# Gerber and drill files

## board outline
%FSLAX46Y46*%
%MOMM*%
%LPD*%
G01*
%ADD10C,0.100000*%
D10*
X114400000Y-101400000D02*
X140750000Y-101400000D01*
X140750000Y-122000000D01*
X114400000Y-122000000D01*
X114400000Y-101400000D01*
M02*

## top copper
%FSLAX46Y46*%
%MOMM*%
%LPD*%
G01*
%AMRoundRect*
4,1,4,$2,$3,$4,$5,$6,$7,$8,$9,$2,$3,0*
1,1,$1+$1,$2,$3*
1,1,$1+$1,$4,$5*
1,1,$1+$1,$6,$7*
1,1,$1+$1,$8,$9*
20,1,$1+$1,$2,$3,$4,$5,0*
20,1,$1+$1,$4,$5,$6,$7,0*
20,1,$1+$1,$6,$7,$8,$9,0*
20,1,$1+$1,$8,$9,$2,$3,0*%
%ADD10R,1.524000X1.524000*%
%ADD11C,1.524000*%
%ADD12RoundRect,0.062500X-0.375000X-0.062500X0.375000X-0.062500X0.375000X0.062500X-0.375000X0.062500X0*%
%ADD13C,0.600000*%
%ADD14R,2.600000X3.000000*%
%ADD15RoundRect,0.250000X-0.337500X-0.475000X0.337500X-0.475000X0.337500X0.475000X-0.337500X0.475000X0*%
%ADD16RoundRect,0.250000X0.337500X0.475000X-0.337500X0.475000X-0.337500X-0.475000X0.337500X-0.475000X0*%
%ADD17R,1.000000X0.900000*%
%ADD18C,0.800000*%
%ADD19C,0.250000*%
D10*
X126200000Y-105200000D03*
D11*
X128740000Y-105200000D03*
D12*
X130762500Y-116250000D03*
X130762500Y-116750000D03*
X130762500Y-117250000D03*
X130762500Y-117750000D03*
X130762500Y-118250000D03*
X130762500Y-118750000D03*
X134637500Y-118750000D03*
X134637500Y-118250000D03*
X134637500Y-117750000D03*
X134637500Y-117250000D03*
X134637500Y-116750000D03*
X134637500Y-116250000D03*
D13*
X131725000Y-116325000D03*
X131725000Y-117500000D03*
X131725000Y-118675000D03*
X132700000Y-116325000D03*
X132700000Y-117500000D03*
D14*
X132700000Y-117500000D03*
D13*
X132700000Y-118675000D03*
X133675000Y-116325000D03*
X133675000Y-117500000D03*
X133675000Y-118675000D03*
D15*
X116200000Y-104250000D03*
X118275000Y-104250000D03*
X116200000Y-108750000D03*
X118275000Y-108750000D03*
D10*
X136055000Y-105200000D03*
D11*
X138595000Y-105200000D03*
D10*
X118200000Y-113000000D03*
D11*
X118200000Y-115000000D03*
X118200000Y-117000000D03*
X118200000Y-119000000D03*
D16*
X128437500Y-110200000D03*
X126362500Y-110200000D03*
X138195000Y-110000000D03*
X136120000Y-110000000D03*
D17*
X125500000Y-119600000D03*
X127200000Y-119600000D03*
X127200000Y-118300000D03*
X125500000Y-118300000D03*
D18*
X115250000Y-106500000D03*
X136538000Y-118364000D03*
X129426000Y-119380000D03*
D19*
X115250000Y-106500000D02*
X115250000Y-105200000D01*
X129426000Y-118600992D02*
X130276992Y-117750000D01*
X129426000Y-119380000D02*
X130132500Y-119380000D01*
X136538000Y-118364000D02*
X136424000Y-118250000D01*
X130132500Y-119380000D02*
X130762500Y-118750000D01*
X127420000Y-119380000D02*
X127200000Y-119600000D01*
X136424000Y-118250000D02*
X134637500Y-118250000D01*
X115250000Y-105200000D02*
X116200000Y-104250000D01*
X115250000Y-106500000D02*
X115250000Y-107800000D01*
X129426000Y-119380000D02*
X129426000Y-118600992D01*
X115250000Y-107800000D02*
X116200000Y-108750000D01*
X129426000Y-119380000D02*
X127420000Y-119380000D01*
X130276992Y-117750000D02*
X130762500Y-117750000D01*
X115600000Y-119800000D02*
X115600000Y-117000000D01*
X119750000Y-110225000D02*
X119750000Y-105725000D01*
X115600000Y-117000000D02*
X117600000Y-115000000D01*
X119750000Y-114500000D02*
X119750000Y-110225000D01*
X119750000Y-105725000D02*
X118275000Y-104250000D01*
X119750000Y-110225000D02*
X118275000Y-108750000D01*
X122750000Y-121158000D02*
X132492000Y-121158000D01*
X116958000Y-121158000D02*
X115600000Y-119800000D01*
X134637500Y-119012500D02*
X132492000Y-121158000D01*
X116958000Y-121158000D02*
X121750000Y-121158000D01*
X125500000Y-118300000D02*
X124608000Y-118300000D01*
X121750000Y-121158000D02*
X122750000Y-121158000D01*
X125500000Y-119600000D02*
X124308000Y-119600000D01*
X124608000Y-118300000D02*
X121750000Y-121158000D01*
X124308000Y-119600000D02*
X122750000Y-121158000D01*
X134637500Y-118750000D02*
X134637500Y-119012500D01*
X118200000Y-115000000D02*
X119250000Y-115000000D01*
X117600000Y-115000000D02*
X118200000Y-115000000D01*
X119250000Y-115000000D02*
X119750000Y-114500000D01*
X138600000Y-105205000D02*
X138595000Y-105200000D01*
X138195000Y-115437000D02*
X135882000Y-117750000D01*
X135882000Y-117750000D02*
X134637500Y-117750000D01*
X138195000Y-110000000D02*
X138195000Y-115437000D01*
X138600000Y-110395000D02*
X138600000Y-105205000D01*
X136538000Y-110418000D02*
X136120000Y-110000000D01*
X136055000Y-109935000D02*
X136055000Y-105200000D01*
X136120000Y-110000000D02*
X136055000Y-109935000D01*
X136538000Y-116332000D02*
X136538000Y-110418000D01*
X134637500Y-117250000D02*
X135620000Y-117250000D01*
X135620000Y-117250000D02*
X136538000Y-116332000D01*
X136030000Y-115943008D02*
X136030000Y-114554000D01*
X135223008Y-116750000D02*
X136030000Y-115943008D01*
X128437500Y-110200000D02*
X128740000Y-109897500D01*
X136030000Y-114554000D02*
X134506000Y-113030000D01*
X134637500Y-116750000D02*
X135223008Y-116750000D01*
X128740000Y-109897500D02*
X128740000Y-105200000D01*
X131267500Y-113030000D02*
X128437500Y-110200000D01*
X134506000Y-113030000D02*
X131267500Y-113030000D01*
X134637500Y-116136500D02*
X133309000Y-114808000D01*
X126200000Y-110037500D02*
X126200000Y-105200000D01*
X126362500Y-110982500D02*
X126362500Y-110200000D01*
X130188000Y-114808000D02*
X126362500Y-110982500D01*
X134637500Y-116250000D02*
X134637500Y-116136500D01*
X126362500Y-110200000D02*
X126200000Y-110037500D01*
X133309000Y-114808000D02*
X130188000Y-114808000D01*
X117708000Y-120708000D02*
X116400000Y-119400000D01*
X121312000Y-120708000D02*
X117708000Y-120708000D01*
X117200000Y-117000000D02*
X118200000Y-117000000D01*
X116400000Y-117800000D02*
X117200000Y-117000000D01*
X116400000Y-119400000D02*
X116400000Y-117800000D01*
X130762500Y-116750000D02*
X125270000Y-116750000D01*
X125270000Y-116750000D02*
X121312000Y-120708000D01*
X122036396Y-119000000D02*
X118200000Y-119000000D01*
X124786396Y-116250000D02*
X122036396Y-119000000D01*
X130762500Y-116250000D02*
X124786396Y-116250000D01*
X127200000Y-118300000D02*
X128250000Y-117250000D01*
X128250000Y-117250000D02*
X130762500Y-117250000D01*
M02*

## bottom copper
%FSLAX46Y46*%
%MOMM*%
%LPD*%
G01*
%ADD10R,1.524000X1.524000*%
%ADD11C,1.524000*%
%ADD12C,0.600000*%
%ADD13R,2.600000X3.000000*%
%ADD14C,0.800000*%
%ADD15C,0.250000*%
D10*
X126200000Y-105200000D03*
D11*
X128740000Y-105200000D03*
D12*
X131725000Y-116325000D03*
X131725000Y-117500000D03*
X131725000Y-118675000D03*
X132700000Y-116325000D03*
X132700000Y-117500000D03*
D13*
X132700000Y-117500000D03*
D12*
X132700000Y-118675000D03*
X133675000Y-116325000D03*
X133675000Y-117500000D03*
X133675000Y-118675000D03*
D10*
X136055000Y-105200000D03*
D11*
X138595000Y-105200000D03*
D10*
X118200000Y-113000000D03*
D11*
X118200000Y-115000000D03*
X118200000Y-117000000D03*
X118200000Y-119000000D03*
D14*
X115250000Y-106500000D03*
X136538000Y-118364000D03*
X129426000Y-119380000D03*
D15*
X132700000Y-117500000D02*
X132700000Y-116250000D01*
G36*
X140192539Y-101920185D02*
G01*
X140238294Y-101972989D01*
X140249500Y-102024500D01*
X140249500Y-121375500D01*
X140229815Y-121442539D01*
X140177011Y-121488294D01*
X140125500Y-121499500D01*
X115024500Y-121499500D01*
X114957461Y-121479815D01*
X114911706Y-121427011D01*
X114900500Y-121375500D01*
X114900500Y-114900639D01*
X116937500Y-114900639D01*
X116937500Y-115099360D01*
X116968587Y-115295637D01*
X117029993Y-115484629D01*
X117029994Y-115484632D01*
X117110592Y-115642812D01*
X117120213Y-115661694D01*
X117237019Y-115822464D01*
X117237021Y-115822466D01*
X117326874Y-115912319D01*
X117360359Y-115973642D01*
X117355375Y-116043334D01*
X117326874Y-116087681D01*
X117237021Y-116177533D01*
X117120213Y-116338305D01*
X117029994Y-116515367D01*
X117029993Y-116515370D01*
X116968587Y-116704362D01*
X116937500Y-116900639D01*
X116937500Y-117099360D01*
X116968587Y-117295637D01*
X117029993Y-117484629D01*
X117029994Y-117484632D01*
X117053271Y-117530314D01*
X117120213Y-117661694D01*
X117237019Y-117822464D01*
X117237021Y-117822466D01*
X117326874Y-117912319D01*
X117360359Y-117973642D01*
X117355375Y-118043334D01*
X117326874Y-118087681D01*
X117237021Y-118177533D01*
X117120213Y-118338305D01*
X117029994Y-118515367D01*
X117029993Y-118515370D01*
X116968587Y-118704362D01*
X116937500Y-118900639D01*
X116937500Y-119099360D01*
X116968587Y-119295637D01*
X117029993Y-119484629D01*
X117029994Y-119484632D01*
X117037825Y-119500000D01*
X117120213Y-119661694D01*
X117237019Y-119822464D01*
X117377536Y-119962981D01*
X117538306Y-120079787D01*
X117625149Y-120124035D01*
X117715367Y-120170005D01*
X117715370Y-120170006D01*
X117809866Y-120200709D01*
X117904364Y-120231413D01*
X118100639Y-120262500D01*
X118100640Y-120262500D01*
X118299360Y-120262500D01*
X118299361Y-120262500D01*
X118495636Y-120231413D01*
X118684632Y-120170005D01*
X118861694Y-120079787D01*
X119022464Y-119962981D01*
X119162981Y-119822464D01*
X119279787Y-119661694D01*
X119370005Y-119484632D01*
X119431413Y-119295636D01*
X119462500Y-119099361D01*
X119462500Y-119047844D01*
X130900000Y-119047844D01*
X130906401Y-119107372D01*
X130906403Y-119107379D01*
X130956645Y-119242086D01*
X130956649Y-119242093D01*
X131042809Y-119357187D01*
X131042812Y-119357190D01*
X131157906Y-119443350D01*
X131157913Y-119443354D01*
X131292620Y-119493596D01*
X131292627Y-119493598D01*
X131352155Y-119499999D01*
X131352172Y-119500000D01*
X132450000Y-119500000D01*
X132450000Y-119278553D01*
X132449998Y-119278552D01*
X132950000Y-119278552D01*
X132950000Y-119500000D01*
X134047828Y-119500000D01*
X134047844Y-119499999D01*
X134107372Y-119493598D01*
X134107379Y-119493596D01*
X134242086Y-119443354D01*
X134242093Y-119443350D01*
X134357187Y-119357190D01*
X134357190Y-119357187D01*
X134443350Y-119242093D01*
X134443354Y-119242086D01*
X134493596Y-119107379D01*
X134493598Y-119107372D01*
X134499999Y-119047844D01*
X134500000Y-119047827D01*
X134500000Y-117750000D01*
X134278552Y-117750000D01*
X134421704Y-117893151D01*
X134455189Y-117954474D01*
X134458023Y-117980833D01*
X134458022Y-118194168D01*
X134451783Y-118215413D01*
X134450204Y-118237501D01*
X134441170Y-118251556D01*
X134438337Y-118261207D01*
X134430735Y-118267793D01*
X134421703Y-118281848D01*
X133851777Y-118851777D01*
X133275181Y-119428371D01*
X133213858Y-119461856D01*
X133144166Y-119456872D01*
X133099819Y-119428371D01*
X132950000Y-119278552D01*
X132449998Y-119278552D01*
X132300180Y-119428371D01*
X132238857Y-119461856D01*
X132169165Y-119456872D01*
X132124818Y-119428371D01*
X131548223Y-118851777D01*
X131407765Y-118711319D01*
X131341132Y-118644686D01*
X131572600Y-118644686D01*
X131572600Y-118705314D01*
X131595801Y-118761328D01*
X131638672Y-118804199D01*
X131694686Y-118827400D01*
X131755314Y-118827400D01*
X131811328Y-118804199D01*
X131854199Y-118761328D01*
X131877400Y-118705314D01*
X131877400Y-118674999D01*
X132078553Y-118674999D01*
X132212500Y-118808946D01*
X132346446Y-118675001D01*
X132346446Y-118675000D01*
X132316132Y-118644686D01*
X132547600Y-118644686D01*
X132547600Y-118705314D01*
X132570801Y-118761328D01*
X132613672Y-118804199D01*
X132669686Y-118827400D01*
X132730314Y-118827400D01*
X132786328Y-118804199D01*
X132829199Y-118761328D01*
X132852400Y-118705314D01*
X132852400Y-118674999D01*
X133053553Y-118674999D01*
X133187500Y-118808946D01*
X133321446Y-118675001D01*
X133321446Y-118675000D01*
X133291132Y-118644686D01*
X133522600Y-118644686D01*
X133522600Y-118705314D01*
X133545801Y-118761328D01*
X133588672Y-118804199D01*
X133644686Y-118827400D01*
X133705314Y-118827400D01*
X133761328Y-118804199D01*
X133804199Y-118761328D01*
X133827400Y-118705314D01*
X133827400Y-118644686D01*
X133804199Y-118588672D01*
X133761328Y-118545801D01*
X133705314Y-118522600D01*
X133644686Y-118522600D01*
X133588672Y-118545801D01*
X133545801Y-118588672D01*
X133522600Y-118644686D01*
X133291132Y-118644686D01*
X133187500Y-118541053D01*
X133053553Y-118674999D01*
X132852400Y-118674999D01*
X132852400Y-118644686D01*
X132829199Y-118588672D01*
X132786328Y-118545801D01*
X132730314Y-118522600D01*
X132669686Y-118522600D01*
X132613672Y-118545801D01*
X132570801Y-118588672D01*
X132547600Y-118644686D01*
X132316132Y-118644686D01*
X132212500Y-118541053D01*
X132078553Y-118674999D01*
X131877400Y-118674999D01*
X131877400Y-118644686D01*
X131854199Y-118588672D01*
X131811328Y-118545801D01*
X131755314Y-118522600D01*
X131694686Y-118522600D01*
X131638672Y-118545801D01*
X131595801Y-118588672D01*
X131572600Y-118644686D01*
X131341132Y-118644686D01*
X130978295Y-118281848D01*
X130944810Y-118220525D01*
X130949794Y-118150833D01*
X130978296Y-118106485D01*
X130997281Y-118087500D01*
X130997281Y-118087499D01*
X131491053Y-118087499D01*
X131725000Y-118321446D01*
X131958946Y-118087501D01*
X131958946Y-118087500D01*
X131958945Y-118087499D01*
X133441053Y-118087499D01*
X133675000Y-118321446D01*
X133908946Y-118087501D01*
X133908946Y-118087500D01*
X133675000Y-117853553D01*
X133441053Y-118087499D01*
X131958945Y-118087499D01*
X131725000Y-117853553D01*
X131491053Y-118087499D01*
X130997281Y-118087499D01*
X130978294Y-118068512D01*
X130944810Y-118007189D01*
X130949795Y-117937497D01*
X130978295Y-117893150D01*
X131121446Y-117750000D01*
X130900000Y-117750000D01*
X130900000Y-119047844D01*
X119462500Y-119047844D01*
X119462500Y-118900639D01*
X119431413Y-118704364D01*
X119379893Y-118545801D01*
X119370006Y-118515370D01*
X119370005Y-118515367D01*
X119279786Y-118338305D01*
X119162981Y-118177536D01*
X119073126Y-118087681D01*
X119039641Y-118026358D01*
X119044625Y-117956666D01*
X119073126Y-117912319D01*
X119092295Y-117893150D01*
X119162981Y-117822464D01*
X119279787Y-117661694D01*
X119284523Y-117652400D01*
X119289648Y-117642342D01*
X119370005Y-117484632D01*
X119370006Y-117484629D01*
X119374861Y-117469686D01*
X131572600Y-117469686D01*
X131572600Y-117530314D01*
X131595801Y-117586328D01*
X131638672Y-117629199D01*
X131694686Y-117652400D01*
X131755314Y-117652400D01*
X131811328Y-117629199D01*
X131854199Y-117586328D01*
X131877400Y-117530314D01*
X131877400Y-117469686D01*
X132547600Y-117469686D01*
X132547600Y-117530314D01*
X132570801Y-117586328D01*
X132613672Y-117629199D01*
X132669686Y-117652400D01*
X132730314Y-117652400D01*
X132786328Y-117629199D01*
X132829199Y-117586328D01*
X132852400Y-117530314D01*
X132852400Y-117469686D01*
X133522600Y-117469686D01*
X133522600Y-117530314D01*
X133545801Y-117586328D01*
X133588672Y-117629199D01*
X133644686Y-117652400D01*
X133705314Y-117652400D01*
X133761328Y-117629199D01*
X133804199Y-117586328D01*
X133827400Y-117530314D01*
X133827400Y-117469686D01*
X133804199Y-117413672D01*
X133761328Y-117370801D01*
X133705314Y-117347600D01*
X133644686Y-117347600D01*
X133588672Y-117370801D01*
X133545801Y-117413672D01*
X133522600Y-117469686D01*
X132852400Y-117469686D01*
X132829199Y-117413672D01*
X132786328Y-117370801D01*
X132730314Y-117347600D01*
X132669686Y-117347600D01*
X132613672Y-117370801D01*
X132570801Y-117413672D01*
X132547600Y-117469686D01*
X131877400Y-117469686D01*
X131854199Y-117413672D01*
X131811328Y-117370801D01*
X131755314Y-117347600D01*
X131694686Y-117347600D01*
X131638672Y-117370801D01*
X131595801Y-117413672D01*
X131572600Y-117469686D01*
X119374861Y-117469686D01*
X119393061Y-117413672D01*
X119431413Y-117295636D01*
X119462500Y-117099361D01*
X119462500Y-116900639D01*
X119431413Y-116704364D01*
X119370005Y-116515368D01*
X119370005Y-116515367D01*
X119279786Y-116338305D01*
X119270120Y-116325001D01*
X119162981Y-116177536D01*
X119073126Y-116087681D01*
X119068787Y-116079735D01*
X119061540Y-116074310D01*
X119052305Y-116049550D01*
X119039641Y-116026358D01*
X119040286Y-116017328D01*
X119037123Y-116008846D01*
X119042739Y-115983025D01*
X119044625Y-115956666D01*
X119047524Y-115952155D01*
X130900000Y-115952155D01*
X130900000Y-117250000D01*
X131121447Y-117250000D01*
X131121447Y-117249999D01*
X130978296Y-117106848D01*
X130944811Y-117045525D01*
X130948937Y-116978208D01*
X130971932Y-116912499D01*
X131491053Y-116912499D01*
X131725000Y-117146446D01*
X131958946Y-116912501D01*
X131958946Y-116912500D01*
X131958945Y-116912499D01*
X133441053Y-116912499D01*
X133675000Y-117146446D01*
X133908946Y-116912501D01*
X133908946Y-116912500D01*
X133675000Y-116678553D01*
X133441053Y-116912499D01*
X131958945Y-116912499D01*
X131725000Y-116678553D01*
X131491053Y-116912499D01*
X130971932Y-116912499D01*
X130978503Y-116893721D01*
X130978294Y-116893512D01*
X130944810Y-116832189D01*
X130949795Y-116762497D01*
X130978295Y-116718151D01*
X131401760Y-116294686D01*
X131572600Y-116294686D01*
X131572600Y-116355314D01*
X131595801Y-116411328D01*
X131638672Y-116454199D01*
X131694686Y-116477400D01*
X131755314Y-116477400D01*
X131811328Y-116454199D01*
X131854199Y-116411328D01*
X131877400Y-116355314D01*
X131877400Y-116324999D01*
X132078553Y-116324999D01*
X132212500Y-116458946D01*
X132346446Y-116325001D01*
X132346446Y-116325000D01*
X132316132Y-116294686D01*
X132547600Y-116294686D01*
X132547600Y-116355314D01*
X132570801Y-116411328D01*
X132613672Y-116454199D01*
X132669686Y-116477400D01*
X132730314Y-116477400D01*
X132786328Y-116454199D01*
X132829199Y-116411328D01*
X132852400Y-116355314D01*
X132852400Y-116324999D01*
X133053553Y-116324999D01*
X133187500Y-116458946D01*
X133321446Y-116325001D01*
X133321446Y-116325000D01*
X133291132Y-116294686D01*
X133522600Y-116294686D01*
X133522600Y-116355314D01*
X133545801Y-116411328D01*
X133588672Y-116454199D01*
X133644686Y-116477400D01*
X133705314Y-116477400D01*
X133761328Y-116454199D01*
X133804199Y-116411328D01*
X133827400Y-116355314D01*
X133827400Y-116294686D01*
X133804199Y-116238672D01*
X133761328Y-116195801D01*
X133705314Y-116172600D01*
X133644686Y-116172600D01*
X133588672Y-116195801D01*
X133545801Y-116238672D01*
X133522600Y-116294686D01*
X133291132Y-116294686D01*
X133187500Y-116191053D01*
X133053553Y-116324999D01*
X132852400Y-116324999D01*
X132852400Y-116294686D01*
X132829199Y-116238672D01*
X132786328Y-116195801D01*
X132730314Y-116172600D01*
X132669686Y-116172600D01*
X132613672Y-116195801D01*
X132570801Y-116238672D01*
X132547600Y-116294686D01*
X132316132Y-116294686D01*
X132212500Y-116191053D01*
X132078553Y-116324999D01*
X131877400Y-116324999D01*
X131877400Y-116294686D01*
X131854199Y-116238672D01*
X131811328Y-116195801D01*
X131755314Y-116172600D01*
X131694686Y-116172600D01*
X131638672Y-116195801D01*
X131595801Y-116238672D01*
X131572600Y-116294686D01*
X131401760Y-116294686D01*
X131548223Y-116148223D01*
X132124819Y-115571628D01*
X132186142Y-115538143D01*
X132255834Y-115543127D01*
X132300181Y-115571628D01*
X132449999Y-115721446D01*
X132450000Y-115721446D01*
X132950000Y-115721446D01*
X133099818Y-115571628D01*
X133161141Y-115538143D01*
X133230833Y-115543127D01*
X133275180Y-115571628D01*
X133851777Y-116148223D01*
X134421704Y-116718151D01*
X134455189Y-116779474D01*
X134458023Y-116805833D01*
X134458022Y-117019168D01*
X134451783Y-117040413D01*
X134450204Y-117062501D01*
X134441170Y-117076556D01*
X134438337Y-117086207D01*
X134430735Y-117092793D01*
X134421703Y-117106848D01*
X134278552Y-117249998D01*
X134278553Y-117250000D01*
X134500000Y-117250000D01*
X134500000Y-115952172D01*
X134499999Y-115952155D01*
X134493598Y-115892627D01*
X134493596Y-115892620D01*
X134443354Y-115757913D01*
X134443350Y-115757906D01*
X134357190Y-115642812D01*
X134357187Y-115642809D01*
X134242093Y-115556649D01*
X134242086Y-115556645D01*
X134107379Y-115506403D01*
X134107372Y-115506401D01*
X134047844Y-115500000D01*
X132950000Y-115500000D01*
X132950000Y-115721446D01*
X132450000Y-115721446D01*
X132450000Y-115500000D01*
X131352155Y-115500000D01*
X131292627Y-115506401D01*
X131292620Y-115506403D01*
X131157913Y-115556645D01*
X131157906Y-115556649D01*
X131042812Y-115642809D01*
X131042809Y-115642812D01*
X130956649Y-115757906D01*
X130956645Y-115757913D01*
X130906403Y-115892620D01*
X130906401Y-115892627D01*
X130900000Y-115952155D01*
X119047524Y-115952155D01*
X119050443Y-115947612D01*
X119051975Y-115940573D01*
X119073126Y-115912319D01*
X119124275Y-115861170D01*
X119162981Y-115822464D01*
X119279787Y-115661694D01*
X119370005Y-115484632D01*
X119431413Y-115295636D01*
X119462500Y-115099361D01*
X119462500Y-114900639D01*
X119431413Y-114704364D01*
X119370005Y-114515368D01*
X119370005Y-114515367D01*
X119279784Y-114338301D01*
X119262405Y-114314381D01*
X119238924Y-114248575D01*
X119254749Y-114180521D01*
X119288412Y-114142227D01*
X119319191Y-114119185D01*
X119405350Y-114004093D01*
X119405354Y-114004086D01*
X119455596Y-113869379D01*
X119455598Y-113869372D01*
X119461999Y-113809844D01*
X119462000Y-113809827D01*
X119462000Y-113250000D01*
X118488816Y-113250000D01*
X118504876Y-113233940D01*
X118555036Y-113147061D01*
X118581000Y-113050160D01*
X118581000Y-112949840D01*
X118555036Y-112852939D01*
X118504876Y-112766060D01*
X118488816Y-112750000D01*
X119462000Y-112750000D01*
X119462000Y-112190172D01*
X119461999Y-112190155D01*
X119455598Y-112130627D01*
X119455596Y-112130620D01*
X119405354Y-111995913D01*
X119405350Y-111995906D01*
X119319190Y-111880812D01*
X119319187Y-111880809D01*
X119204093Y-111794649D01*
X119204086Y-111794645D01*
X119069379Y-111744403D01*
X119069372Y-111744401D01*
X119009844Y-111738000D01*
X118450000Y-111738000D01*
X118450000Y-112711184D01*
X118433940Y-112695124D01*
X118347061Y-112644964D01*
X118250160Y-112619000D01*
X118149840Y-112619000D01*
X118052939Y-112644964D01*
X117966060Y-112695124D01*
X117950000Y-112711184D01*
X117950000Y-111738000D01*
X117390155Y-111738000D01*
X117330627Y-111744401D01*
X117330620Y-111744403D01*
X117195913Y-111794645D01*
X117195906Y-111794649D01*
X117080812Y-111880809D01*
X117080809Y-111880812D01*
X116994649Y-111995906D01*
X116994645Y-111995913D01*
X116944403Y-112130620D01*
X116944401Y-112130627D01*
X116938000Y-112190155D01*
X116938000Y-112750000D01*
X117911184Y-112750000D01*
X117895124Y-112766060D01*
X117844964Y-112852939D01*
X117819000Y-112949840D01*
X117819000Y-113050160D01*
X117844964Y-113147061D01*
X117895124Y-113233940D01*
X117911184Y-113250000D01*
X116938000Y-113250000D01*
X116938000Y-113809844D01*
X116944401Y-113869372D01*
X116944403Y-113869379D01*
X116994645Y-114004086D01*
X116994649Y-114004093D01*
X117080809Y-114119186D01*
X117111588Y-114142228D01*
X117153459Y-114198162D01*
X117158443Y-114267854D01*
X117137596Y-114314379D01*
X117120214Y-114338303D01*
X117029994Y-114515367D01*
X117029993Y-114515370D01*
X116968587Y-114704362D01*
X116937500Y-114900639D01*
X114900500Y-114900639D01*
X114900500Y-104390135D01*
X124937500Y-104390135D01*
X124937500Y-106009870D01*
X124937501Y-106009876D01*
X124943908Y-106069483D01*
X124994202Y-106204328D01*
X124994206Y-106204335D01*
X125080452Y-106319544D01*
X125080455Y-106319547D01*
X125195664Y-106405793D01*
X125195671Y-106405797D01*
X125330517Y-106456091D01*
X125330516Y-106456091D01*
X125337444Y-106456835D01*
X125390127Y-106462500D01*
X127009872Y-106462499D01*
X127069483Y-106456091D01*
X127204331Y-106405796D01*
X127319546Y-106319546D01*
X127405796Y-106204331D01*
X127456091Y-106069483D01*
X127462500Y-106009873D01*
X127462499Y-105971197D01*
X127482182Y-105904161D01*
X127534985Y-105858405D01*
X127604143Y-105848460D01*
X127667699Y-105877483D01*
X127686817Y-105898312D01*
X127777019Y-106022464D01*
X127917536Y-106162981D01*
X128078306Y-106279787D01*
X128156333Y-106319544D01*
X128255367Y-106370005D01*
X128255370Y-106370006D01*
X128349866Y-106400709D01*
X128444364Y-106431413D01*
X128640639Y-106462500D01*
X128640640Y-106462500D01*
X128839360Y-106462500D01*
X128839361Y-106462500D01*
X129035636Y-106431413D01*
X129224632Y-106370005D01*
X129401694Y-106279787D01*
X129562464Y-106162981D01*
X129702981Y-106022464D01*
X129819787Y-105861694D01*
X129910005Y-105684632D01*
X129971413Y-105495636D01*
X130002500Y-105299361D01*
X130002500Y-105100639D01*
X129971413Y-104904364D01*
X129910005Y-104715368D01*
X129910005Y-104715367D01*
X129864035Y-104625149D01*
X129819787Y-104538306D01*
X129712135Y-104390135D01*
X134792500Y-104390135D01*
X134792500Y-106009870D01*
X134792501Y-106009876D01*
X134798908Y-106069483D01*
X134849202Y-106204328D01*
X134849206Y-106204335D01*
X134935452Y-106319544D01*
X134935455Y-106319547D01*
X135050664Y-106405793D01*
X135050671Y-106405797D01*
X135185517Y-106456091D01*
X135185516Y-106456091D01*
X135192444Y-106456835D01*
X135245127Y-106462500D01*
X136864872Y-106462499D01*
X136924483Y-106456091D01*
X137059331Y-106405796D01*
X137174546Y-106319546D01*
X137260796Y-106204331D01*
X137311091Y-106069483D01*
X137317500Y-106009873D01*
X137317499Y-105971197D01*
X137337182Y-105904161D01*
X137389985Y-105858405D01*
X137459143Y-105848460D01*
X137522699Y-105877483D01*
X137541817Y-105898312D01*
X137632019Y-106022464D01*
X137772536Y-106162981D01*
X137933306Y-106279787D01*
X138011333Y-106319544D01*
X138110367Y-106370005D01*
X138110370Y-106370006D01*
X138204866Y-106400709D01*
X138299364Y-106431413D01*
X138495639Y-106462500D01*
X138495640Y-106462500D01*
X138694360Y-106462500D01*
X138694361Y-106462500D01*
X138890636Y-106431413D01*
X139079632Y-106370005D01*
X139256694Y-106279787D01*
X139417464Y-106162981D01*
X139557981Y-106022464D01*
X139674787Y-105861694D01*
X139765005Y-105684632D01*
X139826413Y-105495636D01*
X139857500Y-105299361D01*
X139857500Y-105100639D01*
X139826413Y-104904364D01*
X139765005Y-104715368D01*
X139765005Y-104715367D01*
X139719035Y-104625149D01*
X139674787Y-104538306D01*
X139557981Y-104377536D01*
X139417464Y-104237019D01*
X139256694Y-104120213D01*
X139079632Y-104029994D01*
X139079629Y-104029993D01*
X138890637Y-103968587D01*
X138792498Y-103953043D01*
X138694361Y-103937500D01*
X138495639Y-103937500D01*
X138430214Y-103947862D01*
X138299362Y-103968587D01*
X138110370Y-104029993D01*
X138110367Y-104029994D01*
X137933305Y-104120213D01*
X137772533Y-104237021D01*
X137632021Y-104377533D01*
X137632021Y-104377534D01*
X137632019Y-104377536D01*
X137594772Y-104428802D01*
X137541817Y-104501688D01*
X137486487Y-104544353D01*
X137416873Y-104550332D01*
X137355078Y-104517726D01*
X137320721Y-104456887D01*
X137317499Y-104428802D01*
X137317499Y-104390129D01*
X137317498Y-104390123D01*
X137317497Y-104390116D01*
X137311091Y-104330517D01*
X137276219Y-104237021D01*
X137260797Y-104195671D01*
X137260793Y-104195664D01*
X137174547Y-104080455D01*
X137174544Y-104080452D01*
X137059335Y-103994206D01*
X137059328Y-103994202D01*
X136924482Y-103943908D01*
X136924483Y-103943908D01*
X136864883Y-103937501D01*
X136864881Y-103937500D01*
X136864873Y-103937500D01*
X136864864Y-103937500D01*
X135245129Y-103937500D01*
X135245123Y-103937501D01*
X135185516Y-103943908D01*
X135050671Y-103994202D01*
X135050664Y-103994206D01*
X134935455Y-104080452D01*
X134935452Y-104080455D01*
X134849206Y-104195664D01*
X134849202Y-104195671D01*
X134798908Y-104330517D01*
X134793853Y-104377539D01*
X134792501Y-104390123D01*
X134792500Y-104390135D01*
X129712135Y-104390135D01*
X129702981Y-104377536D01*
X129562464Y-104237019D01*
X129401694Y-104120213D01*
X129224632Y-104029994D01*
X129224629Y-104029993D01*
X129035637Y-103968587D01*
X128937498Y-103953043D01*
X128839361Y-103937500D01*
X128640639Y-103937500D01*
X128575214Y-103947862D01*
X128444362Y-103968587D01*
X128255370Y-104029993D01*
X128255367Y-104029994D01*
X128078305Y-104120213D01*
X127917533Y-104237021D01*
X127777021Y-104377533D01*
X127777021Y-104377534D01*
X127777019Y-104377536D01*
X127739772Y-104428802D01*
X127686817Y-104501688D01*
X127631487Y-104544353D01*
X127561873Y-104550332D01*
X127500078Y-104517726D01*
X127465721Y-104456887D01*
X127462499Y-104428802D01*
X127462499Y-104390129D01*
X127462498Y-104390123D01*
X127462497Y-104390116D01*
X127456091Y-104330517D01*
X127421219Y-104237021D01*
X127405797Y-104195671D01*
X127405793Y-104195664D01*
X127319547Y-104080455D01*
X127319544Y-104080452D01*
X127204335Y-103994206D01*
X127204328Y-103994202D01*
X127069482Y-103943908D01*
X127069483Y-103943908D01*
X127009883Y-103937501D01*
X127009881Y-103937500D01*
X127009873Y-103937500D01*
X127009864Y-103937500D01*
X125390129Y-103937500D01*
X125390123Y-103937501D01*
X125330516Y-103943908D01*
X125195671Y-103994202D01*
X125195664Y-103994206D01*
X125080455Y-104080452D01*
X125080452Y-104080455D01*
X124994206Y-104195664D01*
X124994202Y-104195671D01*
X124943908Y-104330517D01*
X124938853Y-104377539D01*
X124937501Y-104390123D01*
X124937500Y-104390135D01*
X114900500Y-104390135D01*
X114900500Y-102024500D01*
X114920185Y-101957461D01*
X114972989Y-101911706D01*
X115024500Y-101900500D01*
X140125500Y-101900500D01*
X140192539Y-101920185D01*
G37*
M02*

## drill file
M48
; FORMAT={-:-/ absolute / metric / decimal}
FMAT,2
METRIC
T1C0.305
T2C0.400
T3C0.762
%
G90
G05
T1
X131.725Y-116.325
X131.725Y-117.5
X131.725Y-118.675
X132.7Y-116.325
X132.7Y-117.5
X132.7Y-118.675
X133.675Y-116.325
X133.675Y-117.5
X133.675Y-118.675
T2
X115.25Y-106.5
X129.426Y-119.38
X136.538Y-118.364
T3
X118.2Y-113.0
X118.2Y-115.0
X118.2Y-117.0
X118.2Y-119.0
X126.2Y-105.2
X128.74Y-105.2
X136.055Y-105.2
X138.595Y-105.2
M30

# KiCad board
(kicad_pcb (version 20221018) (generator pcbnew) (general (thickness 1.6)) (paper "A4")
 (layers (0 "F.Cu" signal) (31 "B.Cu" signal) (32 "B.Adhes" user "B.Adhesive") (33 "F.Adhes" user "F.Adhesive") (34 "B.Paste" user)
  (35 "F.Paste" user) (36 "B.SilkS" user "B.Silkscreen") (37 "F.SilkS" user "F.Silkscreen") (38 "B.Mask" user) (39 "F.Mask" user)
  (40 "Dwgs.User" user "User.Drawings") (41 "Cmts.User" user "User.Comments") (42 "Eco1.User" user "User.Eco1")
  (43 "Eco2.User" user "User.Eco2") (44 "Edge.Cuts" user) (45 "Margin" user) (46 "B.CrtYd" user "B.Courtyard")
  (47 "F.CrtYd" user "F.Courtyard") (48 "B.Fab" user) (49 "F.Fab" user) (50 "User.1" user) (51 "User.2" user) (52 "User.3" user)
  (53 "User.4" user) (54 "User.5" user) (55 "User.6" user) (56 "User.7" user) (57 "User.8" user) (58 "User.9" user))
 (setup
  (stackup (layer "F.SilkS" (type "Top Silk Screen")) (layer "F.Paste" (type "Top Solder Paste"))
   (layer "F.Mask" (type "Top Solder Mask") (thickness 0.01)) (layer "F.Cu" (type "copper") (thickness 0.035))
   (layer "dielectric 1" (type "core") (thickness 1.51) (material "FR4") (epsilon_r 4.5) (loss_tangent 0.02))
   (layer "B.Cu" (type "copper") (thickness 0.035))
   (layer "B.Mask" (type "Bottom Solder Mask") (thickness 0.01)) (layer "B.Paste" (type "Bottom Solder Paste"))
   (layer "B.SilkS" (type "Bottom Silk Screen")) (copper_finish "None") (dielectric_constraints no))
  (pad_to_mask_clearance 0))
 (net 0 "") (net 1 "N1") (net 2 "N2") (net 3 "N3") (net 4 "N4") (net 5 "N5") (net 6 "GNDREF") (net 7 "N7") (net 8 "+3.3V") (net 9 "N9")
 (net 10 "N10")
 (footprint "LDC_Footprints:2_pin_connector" (layer "F.Cu") (at 127.47 105.2)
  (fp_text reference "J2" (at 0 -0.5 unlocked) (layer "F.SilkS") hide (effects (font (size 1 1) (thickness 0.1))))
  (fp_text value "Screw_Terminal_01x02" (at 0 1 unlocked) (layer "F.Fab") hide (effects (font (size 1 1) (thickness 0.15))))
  (pad "1" thru_hole rect (at -1.27 0) (size 1.524 1.524) (drill 0.762) (layers "*.Cu" "*.Mask") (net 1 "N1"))
  (pad "2" thru_hole circle (at 1.27 0) (size 1.524 1.524) (drill 0.762) (layers "*.Cu" "*.Mask") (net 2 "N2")))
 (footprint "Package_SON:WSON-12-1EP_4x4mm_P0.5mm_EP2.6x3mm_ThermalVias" (layer "F.Cu") (at 132.7 117.5)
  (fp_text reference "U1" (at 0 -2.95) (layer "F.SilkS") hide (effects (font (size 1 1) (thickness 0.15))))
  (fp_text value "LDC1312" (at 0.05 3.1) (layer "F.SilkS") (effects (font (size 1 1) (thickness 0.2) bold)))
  (pad "" smd roundrect (at -0.65 -0.75) (size 1.13 1.3) (layers "F.Paste") (roundrect_rratio 0.221239))
  (pad "" smd roundrect (at -0.65 0.75) (size 1.13 1.3) (layers "F.Paste") (roundrect_rratio 0.221239))
  (pad "" smd roundrect (at 0.65 -0.75) (size 1.13 1.3) (layers "F.Paste") (roundrect_rratio 0.221239))
  (pad "" smd roundrect (at 0.65 0.75) (size 1.13 1.3) (layers "F.Paste") (roundrect_rratio 0.221239))
  (pad "1" smd roundrect (at -1.9375 -1.25) (size 0.875 0.25) (layers "F.Cu" "F.Paste" "F.Mask") (roundrect_rratio 0.25) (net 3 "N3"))
  (pad "2" smd roundrect (at -1.9375 -0.75) (size 0.875 0.25) (layers "F.Cu" "F.Paste" "F.Mask") (roundrect_rratio 0.25) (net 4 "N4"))
  (pad "3" smd roundrect (at -1.9375 -0.25) (size 0.875 0.25) (layers "F.Cu" "F.Paste" "F.Mask") (roundrect_rratio 0.25) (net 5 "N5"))
  (pad "4" smd roundrect (at -1.9375 0.25) (size 0.875 0.25) (layers "F.Cu" "F.Paste" "F.Mask") (roundrect_rratio 0.25) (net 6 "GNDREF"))
  (pad "5" smd roundrect (at -1.9375 0.75) (size 0.875 0.25) (layers "F.Cu" "F.Paste" "F.Mask") (roundrect_rratio 0.25) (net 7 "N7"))
  (pad "6" smd roundrect (at -1.9375 1.25) (size 0.875 0.25) (layers "F.Cu" "F.Paste" "F.Mask") (roundrect_rratio 0.25) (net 6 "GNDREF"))
  (pad "7" smd roundrect (at 1.9375 1.25) (size 0.875 0.25) (layers "F.Cu" "F.Paste" "F.Mask") (roundrect_rratio 0.25) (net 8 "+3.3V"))
  (pad "8" smd roundrect (at 1.9375 0.75) (size 0.875 0.25) (layers "F.Cu" "F.Paste" "F.Mask") (roundrect_rratio 0.25) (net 6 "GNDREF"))
  (pad "9" smd roundrect (at 1.9375 0.25) (size 0.875 0.25) (layers "F.Cu" "F.Paste" "F.Mask") (roundrect_rratio 0.25) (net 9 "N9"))
  (pad "10" smd roundrect (at 1.9375 -0.25) (size 0.875 0.25) (layers "F.Cu" "F.Paste" "F.Mask") (roundrect_rratio 0.25) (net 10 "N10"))
  (pad "11" smd roundrect (at 1.9375 -0.75) (size 0.875 0.25) (layers "F.Cu" "F.Paste" "F.Mask") (roundrect_rratio 0.25) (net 2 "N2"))
  (pad "12" smd roundrect (at 1.9375 -1.25) (size 0.875 0.25) (layers "F.Cu" "F.Paste" "F.Mask") (roundrect_rratio 0.25) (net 1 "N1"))
  (pad "13" thru_hole circle (at -0.975 -1.175) (size 0.6 0.6) (drill 0.3048) (layers "*.Cu") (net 6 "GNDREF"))
  (pad "13" thru_hole circle (at -0.975 0) (size 0.6 0.6) (drill 0.3048) (layers "*.Cu") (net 6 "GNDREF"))
  (pad "13" thru_hole circle (at -0.975 1.175) (size 0.6 0.6) (drill 0.3048) (layers "*.Cu") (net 6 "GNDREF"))
  (pad "13" thru_hole circle (at 0 -1.175) (size 0.6 0.6) (drill 0.3048) (layers "*.Cu") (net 6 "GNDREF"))
  (pad "13" thru_hole circle (at 0 0) (size 0.6 0.6) (drill 0.3048) (layers "*.Cu") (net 6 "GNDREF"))
  (pad "13" smd rect (at 0 0) (size 2.6 3) (layers "F.Cu" "F.Mask") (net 6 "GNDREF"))
  (pad "13" smd rect (at 0 0) (size 2.6 3) (layers "B.Cu") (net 6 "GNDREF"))
  (pad "13" thru_hole circle (at 0 1.175) (size 0.6 0.6) (drill 0.3048) (layers "*.Cu") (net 6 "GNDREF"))
  (pad "13" thru_hole circle (at 0.975 -1.175) (size 0.6 0.6) (drill 0.3048) (layers "*.Cu") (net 6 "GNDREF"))
  (pad "13" thru_hole circle (at 0.975 0) (size 0.6 0.6) (drill 0.3048) (layers "*.Cu") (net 6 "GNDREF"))
  (pad "13" thru_hole circle (at 0.975 1.175) (size 0.6 0.6) (drill 0.3048) (layers "*.Cu") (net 6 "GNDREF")))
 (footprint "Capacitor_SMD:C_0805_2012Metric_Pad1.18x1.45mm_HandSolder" (layer "F.Cu") (at 117.2375 104.25)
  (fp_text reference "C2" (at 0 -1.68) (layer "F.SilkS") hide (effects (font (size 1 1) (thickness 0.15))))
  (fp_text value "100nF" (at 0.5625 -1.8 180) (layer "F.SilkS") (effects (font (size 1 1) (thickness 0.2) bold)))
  (pad "1" smd roundrect (at -1.0375 0) (size 1.175 1.45) (layers "F.Cu" "F.Paste" "F.Mask") (roundrect_rratio 0.212766) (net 6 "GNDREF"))
  (pad "2" smd roundrect (at 1.0375 0) (size 1.175 1.45) (layers "F.Cu" "F.Paste" "F.Mask") (roundrect_rratio 0.212766) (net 8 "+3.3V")))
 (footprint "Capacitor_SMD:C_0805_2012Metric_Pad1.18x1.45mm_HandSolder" (layer "F.Cu") (at 117.2375 108.75)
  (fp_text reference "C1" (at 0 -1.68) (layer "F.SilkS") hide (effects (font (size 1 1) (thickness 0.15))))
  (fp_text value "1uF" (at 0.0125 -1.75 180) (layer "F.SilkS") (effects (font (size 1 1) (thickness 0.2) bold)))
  (pad "1" smd roundrect (at -1.0375 0) (size 1.175 1.45) (layers "F.Cu" "F.Paste" "F.Mask") (roundrect_rratio 0.212766) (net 6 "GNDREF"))
  (pad "2" smd roundrect (at 1.0375 0) (size 1.175 1.45) (layers "F.Cu" "F.Paste" "F.Mask") (roundrect_rratio 0.212766) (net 8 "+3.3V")))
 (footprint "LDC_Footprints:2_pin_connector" (layer "F.Cu") (at 137.325 105.2)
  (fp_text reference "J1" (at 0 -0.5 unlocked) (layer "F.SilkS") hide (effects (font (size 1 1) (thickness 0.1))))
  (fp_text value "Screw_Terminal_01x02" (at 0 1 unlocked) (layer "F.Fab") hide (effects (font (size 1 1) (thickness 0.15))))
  (pad "1" thru_hole rect (at -1.27 0) (size 1.524 1.524) (drill 0.762) (layers "*.Cu" "*.Mask") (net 10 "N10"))
  (pad "2" thru_hole circle (at 1.27 0) (size 1.524 1.524) (drill 0.762) (layers "*.Cu" "*.Mask") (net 9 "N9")))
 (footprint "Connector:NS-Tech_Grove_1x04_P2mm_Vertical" (layer "F.Cu") (at 118.2 113)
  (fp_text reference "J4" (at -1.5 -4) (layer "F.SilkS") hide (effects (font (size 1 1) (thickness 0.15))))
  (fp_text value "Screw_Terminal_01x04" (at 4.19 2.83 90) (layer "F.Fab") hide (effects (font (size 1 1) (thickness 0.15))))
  (pad "1" thru_hole rect (at 0 0) (size 1.524 1.524) (drill 0.762) (layers "*.Cu" "*.Mask") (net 6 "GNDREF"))
  (pad "2" thru_hole circle (at 0 2) (size 1.524 1.524) (drill 0.762) (layers "*.Cu" "*.Mask") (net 8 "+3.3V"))
  (pad "3" thru_hole circle (at 0 4) (size 1.524 1.524) (drill 0.762) (layers "*.Cu" "*.Mask") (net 4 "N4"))
  (pad "4" thru_hole circle (at 0 6) (size 1.524 1.524) (drill 0.762) (layers "*.Cu" "*.Mask") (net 3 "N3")))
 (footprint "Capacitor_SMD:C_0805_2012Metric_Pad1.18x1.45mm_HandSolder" (layer "F.Cu") (at 127.4 110.2 180)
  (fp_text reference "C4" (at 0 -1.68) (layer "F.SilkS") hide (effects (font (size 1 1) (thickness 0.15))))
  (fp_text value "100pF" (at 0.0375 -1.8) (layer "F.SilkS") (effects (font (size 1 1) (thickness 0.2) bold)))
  (pad "1" smd roundrect (at -1.0375 0 180) (size 1.175 1.45) (layers "F.Cu" "F.Paste" "F.Mask") (roundrect_rratio 0.212766) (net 2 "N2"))
  (pad "2" smd roundrect (at 1.0375 0 180) (size 1.175 1.45) (layers "F.Cu" "F.Paste" "F.Mask") (roundrect_rratio 0.212766) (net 1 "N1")))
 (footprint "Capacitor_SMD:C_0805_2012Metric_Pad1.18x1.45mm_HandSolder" (layer "F.Cu") (at 137.1575 110 180)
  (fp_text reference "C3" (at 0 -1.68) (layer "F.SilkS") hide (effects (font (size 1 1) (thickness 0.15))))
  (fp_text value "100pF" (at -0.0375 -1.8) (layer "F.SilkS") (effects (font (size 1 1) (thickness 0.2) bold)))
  (pad "1" smd roundrect (at -1.0375 0 180) (size 1.175 1.45) (layers "F.Cu" "F.Paste" "F.Mask") (roundrect_rratio 0.212766) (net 9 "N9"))
  (pad "2" smd roundrect (at 1.0375 0 180) (size 1.175 1.45) (layers "F.Cu" "F.Paste" "F.Mask") (roundrect_rratio 0.212766) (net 10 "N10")))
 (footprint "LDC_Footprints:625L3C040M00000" (layer "F.Cu") (at 126.35 118.95)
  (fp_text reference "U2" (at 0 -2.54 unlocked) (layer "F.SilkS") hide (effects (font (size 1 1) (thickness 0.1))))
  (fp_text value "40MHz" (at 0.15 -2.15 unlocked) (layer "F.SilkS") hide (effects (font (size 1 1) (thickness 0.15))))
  (pad "1" smd rect (at -0.85 0.65) (size 1 0.9) (layers "F.Cu" "F.Paste" "F.Mask") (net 8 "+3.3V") (thermal_bridge_angle 45))
  (pad "2" smd rect (at 0.85 0.65) (size 1 0.9) (layers "F.Cu" "F.Paste" "F.Mask") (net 6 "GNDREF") (thermal_bridge_angle 45))
  (pad "3" smd rect (at 0.85 -0.65) (size 1 0.9) (layers "F.Cu" "F.Paste" "F.Mask") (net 5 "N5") (thermal_bridge_angle 45))
  (pad "4" smd rect (at -0.85 -0.65) (size 1 0.9) (layers "F.Cu" "F.Paste" "F.Mask") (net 8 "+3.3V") (thermal_bridge_angle 45)))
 (gr_rect (start 114.4 101.4) (end 140.75 122) (stroke (width 0.1) (type solid)) (fill none) (layer "Edge.Cuts"))
 (segment (start 115.25 106.5) (end 115.25 105.2) (width 0.25) (layer "F.Cu") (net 6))
 (segment (start 129.426 118.600992) (end 130.276992 117.75) (width 0.25) (layer "F.Cu") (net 6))
 (segment (start 129.426 119.38) (end 130.1325 119.38) (width 0.25) (layer "F.Cu") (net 6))
 (segment (start 136.538 118.364) (end 136.424 118.25) (width 0.25) (layer "F.Cu") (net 6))
 (segment (start 130.1325 119.38) (end 130.7625 118.75) (width 0.25) (layer "F.Cu") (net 6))
 (segment (start 127.42 119.38) (end 127.2 119.6) (width 0.25) (layer "F.Cu") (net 6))
 (segment (start 136.424 118.25) (end 134.6375 118.25) (width 0.25) (layer "F.Cu") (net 6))
 (segment (start 115.25 105.2) (end 116.2 104.25) (width 0.25) (layer "F.Cu") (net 6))
 (segment (start 115.25 106.5) (end 115.25 107.8) (width 0.25) (layer "F.Cu") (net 6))
 (segment (start 129.426 119.38) (end 129.426 118.600992) (width 0.25) (layer "F.Cu") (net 6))
 (segment (start 115.25 107.8) (end 116.2 108.75) (width 0.25) (layer "F.Cu") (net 6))
 (segment (start 129.426 119.38) (end 127.42 119.38) (width 0.25) (layer "F.Cu") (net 6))
 (segment (start 130.276992 117.75) (end 130.7625 117.75) (width 0.25) (layer "F.Cu") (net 6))
 (via (at 115.25 106.5) (size 0.8) (drill 0.4) (layers "F.Cu" "B.Cu") (free) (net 6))
 (via (at 136.538 118.364) (size 0.8) (drill 0.4) (layers "F.Cu" "B.Cu") (free) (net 6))
 (via (at 129.426 119.38) (size 0.8) (drill 0.4) (layers "F.Cu" "B.Cu") (free) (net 6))
 (segment (start 132.7 117.5) (end 132.7 116.25) (width 0.25) (layer "B.Cu") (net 6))
 (segment (start 115.6 119.8) (end 115.6 117) (width 0.25) (layer "F.Cu") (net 8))
 (segment (start 119.75 110.225) (end 119.75 105.725) (width 0.25) (layer "F.Cu") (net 8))
 (segment (start 115.6 117) (end 117.6 115) (width 0.25) (layer "F.Cu") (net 8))
 (segment (start 119.75 114.5) (end 119.75 110.225) (width 0.25) (layer "F.Cu") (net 8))
 (segment (start 119.75 105.725) (end 118.275 104.25) (width 0.25) (layer "F.Cu") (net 8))
 (segment (start 119.75 110.225) (end 118.275 108.75) (width 0.25) (layer "F.Cu") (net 8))
 (segment (start 122.75 121.158) (end 132.492 121.158) (width 0.25) (layer "F.Cu") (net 8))
 (segment (start 116.958 121.158) (end 115.6 119.8) (width 0.25) (layer "F.Cu") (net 8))
 (segment (start 134.6375 119.0125) (end 132.492 121.158) (width 0.25) (layer "F.Cu") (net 8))
 (segment (start 116.958 121.158) (end 121.75 121.158) (width 0.25) (layer "F.Cu") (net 8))
 (segment (start 125.5 118.3) (end 124.608 118.3) (width 0.25) (layer "F.Cu") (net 8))
 (segment (start 121.75 121.158) (end 122.75 121.158) (width 0.25) (layer "F.Cu") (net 8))
 (segment (start 125.5 119.6) (end 124.308 119.6) (width 0.25) (layer "F.Cu") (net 8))
 (segment (start 124.608 118.3) (end 121.75 121.158) (width 0.25) (layer "F.Cu") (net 8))
 (segment (start 124.308 119.6) (end 122.75 121.158) (width 0.25) (layer "F.Cu") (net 8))
 (segment (start 134.6375 118.75) (end 134.6375 119.0125) (width 0.25) (layer "F.Cu") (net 8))
 (segment (start 118.2 115) (end 119.25 115) (width 0.25) (layer "F.Cu") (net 8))
 (segment (start 117.6 115) (end 118.2 115) (width 0.25) (layer "F.Cu") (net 8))
 (segment (start 119.25 115) (end 119.75 114.5) (width 0.25) (layer "F.Cu") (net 8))
 (segment (start 138.6 105.205) (end 138.595 105.2) (width 0.25) (layer "F.Cu") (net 9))
 (segment (start 138.195 115.437) (end 135.882 117.75) (width 0.25) (layer "F.Cu") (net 9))
 (segment (start 135.882 117.75) (end 134.6375 117.75) (width 0.25) (layer "F.Cu") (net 9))
 (segment (start 138.195 110) (end 138.195 115.437) (width 0.25) (layer "F.Cu") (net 9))
 (segment (start 138.6 110.395) (end 138.6 105.205) (width 0.25) (layer "F.Cu") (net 9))
 (segment (start 136.538 110.418) (end 136.12 110) (width 0.25) (layer "F.Cu") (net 10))
 (segment (start 136.055 109.935) (end 136.055 105.2) (width 0.25) (layer "F.Cu") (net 10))
 (segment (start 136.12 110) (end 136.055 109.935) (width 0.25) (layer "F.Cu") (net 10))
 (segment (start 136.538 116.332) (end 136.538 110.418) (width 0.25) (layer "F.Cu") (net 10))
 (segment (start 134.6375 117.25) (end 135.62 117.25) (width 0.25) (layer "F.Cu") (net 10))
 (segment (start 135.62 117.25) (end 136.538 116.332) (width 0.25) (layer "F.Cu") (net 10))
 (segment (start 136.03 115.943008) (end 136.03 114.554) (width 0.25) (layer "F.Cu") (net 2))
 (segment (start 135.223008 116.75) (end 136.03 115.943008) (width 0.25) (layer "F.Cu") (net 2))
 (segment (start 128.4375 110.2) (end 128.74 109.8975) (width 0.25) (layer "F.Cu") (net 2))
 (segment (start 136.03 114.554) (end 134.506 113.03) (width 0.25) (layer "F.Cu") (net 2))
 (segment (start 134.6375 116.75) (end 135.223008 116.75) (width 0.25) (layer "F.Cu") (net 2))
 (segment (start 128.74 109.8975) (end 128.74 105.2) (width 0.25) (layer "F.Cu") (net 2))
 (segment (start 131.2675 113.03) (end 128.4375 110.2) (width 0.25) (layer "F.Cu") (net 2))
 (segment (start 134.506 113.03) (end 131.2675 113.03) (width 0.25) (layer "F.Cu") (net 2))
 (segment (start 134.6375 116.1365) (end 133.309 114.808) (width 0.25) (layer "F.Cu") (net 1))
 (segment (start 126.2 110.0375) (end 126.2 105.2) (width 0.25) (layer "F.Cu") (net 1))
 (segment (start 126.3625 110.9825) (end 126.3625 110.2) (width 0.25) (layer "F.Cu") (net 1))
 (segment (start 130.188 114.808) (end 126.3625 110.9825) (width 0.25) (layer "F.Cu") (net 1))
 (segment (start 134.6375 116.25) (end 134.6375 116.1365) (width 0.25) (layer "F.Cu") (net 1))
 (segment (start 126.3625 110.2) (end 126.2 110.0375) (width 0.25) (layer "F.Cu") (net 1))
 (segment (start 133.309 114.808) (end 130.188 114.808) (width 0.25) (layer "F.Cu") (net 1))
 (segment (start 117.708 120.708) (end 116.4 119.4) (width 0.25) (layer "F.Cu") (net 4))
 (segment (start 121.312 120.708) (end 117.708 120.708) (width 0.25) (layer "F.Cu") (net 4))
 (segment (start 117.2 117) (end 118.2 117) (width 0.25) (layer "F.Cu") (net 4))
 (segment (start 116.4 117.8) (end 117.2 117) (width 0.25) (layer "F.Cu") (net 4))
 (segment (start 116.4 119.4) (end 116.4 117.8) (width 0.25) (layer "F.Cu") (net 4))
 (segment (start 130.7625 116.75) (end 125.27 116.75) (width 0.25) (layer "F.Cu") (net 4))
 (segment (start 125.27 116.75) (end 121.312 120.708) (width 0.25) (layer "F.Cu") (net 4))
 (segment (start 122.036396 119) (end 118.2 119) (width 0.25) (layer "F.Cu") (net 3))
 (segment (start 124.786396 116.25) (end 122.036396 119) (width 0.25) (layer "F.Cu") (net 3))
 (segment (start 130.7625 116.25) (end 124.786396 116.25) (width 0.25) (layer "F.Cu") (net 3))
 (segment (start 127.2 118.3) (end 128.25 117.25) (width 0.25) (layer "F.Cu") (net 5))
 (segment (start 128.25 117.25) (end 130.7625 117.25) (width 0.25) (layer "F.Cu") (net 5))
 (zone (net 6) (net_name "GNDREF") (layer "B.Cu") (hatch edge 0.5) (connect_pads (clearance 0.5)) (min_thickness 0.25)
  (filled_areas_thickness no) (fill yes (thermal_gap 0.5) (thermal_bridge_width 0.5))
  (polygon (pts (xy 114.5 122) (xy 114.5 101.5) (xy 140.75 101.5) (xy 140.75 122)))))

